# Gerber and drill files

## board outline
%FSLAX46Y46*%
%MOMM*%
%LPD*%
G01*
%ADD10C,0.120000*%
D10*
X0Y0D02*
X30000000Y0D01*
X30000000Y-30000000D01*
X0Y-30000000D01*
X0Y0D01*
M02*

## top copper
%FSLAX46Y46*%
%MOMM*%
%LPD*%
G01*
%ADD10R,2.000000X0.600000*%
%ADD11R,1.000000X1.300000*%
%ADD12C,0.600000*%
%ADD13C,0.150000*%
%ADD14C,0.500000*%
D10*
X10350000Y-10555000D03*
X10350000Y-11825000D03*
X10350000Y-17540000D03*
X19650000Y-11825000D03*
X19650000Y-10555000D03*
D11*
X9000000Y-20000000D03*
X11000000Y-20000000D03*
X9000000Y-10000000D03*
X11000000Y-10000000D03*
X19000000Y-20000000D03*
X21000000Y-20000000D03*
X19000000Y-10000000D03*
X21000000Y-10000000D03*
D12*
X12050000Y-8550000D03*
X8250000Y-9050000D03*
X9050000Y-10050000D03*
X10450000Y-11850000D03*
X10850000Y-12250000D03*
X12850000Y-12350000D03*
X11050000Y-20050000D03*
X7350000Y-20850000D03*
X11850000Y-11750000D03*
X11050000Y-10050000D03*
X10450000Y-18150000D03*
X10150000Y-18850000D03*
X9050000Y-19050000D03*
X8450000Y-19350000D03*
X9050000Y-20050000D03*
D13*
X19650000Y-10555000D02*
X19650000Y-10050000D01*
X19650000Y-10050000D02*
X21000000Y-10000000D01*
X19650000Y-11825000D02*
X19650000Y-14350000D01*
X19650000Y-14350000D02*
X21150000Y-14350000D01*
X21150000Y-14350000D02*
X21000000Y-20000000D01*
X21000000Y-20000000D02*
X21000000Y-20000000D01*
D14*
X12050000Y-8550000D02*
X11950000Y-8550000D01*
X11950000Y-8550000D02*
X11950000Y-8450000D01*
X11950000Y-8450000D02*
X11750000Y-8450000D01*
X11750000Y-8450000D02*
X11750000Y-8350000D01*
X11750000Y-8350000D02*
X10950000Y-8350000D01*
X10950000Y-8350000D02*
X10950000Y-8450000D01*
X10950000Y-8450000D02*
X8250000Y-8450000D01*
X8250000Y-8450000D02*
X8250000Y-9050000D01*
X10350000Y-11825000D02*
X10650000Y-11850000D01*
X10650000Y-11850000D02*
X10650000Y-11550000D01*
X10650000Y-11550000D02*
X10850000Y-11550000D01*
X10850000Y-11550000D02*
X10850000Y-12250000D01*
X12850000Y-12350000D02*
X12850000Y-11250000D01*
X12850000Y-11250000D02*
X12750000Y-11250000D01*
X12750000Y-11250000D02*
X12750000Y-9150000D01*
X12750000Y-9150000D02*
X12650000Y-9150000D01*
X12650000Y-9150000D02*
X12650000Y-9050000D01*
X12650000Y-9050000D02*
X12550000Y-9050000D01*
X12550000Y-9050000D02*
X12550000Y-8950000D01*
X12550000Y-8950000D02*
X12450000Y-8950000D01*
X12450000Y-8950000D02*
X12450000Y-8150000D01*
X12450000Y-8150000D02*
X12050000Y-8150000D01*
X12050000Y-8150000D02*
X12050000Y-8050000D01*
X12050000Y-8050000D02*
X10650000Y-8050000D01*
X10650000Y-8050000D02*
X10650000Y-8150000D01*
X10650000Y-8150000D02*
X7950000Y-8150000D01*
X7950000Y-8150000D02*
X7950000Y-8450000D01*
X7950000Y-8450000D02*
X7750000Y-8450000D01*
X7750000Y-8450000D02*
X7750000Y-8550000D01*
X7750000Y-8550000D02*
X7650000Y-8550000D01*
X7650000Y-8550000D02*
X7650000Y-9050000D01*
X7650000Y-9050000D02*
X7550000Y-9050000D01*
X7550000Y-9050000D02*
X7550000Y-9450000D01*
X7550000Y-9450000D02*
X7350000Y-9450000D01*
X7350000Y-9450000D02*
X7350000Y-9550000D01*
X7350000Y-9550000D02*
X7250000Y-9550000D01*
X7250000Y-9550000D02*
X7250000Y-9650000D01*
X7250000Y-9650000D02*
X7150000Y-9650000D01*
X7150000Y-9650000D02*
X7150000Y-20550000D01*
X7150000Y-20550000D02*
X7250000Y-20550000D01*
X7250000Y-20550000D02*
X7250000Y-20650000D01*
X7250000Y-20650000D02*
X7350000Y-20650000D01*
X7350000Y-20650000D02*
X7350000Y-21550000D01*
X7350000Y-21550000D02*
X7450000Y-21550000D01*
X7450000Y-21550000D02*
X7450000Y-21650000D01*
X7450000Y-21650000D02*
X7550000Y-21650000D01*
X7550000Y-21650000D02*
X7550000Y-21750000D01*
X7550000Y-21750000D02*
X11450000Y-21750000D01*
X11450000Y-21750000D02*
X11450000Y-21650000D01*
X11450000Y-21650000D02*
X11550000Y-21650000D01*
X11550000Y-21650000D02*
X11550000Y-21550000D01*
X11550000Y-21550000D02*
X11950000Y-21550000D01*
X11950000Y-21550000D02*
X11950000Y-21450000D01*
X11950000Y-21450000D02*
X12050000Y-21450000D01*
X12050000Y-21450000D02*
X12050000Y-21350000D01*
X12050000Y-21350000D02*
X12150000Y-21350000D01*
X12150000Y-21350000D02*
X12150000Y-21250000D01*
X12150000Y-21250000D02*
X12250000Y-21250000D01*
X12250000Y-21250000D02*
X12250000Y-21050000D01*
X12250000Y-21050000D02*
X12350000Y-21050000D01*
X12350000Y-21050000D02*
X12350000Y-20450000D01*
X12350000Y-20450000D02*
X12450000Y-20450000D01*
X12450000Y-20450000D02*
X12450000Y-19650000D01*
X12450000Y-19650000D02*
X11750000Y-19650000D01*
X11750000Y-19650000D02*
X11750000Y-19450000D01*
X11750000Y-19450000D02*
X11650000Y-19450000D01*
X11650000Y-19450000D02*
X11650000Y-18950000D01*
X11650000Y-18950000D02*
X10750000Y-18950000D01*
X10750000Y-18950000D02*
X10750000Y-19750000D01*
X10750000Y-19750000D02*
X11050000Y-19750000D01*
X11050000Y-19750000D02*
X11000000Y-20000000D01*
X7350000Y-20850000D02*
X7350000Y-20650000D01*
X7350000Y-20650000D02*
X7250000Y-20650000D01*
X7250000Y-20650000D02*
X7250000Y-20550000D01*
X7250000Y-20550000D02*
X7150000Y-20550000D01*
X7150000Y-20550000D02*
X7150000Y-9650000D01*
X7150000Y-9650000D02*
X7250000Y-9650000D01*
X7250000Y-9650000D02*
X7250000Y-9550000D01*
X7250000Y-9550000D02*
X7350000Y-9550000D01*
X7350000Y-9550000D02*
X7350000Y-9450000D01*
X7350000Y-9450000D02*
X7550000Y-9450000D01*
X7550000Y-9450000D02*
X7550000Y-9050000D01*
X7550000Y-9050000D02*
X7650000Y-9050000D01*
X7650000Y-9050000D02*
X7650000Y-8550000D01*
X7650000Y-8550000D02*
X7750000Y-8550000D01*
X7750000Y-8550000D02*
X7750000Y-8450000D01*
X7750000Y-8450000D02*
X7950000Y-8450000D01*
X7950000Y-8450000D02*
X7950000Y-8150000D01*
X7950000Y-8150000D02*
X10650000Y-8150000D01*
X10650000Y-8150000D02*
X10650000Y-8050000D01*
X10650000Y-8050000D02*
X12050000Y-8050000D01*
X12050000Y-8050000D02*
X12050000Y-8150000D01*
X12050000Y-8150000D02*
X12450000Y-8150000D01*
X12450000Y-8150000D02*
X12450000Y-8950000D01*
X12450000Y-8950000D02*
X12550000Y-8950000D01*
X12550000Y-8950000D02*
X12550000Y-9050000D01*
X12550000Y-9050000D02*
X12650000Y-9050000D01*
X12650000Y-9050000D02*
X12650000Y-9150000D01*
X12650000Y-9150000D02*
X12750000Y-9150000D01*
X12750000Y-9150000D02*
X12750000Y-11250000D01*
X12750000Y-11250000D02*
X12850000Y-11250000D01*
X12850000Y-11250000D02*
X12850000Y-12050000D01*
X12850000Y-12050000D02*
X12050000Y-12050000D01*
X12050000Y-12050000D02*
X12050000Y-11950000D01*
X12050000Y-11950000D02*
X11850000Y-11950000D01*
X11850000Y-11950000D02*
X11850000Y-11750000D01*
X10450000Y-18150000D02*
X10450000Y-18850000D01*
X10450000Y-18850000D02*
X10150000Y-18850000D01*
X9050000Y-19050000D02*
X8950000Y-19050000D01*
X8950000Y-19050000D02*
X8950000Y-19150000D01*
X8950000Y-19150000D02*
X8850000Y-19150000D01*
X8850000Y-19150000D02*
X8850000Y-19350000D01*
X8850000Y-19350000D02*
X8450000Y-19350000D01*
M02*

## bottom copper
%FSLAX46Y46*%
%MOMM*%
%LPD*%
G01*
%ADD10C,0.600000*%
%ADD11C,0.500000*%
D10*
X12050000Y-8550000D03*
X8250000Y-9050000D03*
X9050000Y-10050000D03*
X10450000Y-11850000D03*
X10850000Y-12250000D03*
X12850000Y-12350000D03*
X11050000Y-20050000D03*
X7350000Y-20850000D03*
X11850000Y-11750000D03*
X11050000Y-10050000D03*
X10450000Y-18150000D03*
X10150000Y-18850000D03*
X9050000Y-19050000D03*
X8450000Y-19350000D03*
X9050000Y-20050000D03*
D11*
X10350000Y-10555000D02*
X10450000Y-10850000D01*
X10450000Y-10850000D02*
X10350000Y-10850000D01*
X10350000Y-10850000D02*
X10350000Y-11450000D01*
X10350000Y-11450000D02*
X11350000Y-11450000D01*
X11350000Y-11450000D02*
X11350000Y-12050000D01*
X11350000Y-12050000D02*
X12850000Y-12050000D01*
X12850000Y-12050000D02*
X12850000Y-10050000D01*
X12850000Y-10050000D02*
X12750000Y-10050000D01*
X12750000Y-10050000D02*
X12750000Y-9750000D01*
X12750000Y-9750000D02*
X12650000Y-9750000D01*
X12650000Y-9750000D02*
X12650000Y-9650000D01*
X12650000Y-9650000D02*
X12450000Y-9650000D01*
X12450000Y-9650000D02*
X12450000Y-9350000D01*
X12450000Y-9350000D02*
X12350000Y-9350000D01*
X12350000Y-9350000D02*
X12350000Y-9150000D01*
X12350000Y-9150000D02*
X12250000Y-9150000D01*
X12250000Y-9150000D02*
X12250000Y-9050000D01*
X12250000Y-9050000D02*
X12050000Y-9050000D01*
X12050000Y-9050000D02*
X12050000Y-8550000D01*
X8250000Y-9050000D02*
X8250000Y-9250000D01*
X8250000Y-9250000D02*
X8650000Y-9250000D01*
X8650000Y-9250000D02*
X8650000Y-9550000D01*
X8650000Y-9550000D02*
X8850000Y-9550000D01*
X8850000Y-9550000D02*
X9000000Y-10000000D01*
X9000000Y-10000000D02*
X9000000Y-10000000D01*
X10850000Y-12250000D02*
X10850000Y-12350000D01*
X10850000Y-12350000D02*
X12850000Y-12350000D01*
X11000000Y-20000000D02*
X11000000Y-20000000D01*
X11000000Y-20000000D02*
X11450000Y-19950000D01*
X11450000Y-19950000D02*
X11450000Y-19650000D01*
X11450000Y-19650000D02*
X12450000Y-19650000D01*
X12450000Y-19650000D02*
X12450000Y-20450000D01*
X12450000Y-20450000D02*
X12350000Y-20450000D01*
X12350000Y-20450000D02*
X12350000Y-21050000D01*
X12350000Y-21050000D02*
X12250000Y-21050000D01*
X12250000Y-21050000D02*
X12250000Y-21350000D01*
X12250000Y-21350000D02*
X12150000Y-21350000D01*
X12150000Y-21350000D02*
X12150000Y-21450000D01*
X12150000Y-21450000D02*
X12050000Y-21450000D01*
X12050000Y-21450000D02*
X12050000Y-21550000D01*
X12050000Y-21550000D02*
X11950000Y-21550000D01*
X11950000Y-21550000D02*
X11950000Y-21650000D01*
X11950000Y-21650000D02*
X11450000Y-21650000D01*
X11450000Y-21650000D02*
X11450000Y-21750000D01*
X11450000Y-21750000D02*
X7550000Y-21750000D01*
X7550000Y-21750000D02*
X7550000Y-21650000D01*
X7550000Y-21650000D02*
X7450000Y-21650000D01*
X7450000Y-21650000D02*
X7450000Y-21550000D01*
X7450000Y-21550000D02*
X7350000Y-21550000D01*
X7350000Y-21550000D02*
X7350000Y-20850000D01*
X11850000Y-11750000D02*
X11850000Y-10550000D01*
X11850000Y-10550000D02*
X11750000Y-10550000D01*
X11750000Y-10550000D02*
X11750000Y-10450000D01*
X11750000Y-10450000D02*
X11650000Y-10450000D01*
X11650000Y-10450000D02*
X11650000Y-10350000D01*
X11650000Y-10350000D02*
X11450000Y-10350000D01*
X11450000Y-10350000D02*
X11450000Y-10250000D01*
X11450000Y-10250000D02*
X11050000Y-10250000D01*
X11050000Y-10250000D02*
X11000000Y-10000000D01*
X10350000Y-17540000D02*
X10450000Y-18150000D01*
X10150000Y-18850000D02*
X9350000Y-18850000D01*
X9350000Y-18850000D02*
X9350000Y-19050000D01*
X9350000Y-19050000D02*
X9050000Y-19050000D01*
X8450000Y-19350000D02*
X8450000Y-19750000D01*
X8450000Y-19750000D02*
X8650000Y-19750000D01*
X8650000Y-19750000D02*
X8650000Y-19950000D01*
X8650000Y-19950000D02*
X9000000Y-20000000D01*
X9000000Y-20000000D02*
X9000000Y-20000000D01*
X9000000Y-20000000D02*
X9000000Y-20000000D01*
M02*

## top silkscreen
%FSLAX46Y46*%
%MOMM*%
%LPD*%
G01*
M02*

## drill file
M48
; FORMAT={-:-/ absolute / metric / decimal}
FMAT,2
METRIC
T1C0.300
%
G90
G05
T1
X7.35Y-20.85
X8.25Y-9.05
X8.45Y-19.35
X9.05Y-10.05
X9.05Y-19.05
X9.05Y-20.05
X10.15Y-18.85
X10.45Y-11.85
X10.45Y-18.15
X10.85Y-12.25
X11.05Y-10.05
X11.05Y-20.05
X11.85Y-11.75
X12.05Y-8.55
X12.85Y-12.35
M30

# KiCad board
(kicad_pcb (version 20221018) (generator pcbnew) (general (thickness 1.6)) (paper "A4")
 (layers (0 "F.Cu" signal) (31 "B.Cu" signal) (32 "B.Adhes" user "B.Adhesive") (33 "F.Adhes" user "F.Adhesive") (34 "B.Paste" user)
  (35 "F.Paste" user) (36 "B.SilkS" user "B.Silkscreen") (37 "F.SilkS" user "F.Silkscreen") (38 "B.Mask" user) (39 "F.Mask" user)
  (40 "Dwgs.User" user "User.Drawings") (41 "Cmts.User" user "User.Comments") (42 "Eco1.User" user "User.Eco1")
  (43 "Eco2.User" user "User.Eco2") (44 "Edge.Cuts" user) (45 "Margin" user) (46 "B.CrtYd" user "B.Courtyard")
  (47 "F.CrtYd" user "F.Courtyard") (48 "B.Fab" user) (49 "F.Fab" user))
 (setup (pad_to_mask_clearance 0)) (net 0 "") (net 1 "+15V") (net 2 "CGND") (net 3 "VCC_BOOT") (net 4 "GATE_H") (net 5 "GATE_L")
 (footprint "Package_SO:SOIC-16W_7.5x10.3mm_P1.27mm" (layer "F.Cu") (at 15 14.999999656677247 0) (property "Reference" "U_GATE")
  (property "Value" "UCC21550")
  (pad "1" smd rect (at -4.65 -4.445) (size 2 0.6) (layers "F.Cu" "F.Paste" "F.Mask") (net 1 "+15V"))
  (pad "2" smd rect (at -4.65 -3.175) (size 2 0.6) (layers "F.Cu" "F.Paste" "F.Mask") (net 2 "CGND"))
  (pad "7" smd rect (at -4.65 2.54) (size 2 0.6) (layers "F.Cu" "F.Paste" "F.Mask") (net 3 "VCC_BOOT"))
  (pad "14" smd rect (at 4.65 -3.175) (size 2 0.6) (layers "F.Cu" "F.Paste" "F.Mask") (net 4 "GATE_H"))
  (pad "16" smd rect (at 4.65 -4.445) (size 2 0.6) (layers "F.Cu" "F.Paste" "F.Mask") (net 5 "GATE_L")))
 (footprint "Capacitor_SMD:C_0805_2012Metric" (layer "F.Cu") (at 10 20 0) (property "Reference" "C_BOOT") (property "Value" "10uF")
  (pad "1" smd rect (at -1 0) (size 1 1.3) (layers "F.Cu" "F.Paste" "F.Mask") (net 3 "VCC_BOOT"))
  (pad "2" smd rect (at 1 0) (size 1 1.3) (layers "F.Cu" "F.Paste" "F.Mask") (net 2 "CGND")))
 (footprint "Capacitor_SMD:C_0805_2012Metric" (layer "F.Cu") (at 10 10 0) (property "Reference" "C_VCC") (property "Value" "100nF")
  (pad "1" smd rect (at -1 0) (size 1 1.3) (layers "F.Cu" "F.Paste" "F.Mask") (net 1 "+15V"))
  (pad "2" smd rect (at 1 0) (size 1 1.3) (layers "F.Cu" "F.Paste" "F.Mask") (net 2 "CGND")))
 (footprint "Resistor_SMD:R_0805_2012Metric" (layer "F.Cu") (at 20 20 0) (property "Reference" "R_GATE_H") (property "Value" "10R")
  (pad "1" smd rect (at -1 0) (size 1 1.3) (layers "F.Cu" "F.Paste" "F.Mask") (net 4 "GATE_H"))
  (pad "2" smd rect (at 1 0) (size 1 1.3) (layers "F.Cu" "F.Paste" "F.Mask") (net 4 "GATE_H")))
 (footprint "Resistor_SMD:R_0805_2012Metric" (layer "F.Cu") (at 20 10 0) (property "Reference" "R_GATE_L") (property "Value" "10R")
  (pad "1" smd rect (at -1 0) (size 1 1.3) (layers "F.Cu" "F.Paste" "F.Mask") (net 5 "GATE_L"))
  (pad "2" smd rect (at 1 0) (size 1 1.3) (layers "F.Cu" "F.Paste" "F.Mask") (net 5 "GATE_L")))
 (gr_rect (start 0 0) (end 30 30) (layer "Edge.Cuts") (width 0.12))
 (segment (start 19.65 10.554999656677246) (end 19.650000000000002 10.05) (width 0.15) (layer "F.Cu") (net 5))
 (segment (start 19.650000000000002 10.05) (end 21.0 10.0) (width 0.15) (layer "F.Cu") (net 5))
 (segment (start 19.65 11.824999656677246) (end 19.650000000000002 14.350000000000001) (width 0.15) (layer "F.Cu") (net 4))
 (segment (start 19.650000000000002 14.350000000000001) (end 21.150000000000002 14.350000000000001) (width 0.15) (layer "F.Cu") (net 4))
 (segment (start 21.150000000000002 14.350000000000001) (end 21.0 20.0) (width 0.15) (layer "F.Cu") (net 4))
 (segment (start 21.0 20.0) (end 21.0 20.0) (width 0.15) (layer "F.Cu") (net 4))
 (segment (start 10.35 10.554999656677246) (end 10.450000000000001 10.850000000000001) (width 0.5) (layer "B.Cu") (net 1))
 (segment (start 10.450000000000001 10.850000000000001) (end 10.350000000000001 10.850000000000001) (width 0.5) (layer "B.Cu") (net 1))
 (segment (start 10.350000000000001 10.850000000000001) (end 10.350000000000001 11.450000000000001) (width 0.5) (layer "B.Cu") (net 1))
 (segment (start 10.350000000000001 11.450000000000001) (end 11.350000000000001 11.450000000000001) (width 0.5) (layer "B.Cu") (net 1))
 (segment (start 11.350000000000001 11.450000000000001) (end 11.350000000000001 12.05) (width 0.5) (layer "B.Cu") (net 1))
 (segment (start 11.350000000000001 12.05) (end 12.850000000000001 12.05) (width 0.5) (layer "B.Cu") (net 1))
 (segment (start 12.850000000000001 12.05) (end 12.850000000000001 10.05) (width 0.5) (layer "B.Cu") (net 1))
 (segment (start 12.850000000000001 10.05) (end 12.750000000000002 10.05) (width 0.5) (layer "B.Cu") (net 1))
 (segment (start 12.750000000000002 10.05) (end 12.750000000000002 9.750000000000002) (width 0.5) (layer "B.Cu") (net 1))
 (segment (start 12.750000000000002 9.750000000000002) (end 12.650000000000002 9.750000000000002) (width 0.5) (layer "B.Cu") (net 1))
 (segment (start 12.650000000000002 9.750000000000002) (end 12.650000000000002 9.650000000000002) (width 0.5) (layer "B.Cu") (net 1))
 (segment (start 12.650000000000002 9.650000000000002) (end 12.450000000000001 9.650000000000002) (width 0.5) (layer "B.Cu") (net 1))
 (segment (start 12.450000000000001 9.650000000000002) (end 12.450000000000001 9.350000000000001) (width 0.5) (layer "B.Cu") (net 1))
 (segment (start 12.450000000000001 9.350000000000001) (end 12.350000000000001 9.350000000000001) (width 0.5) (layer "B.Cu") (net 1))
 (segment (start 12.350000000000001 9.350000000000001) (end 12.350000000000001 9.15) (width 0.5) (layer "B.Cu") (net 1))
 (segment (start 12.350000000000001 9.15) (end 12.250000000000002 9.15) (width 0.5) (layer "B.Cu") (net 1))
 (segment (start 12.250000000000002 9.15) (end 12.250000000000002 9.05) (width 0.5) (layer "B.Cu") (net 1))
 (segment (start 12.250000000000002 9.05) (end 12.05 9.05) (width 0.5) (layer "B.Cu") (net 1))
 (segment (start 12.05 9.05) (end 12.05 8.55) (width 0.5) (layer "B.Cu") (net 1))
 (segment (start 12.05 8.55) (end 11.950000000000001 8.55) (width 0.5) (layer "F.Cu") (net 1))
 (segment (start 11.950000000000001 8.55) (end 11.950000000000001 8.450000000000001) (width 0.5) (layer "F.Cu") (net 1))
 (segment (start 11.950000000000001 8.450000000000001) (end 11.750000000000002 8.450000000000001) (width 0.5) (layer "F.Cu") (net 1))
 (segment (start 11.750000000000002 8.450000000000001) (end 11.750000000000002 8.350000000000001) (width 0.5) (layer "F.Cu") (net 1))
 (segment (start 11.750000000000002 8.350000000000001) (end 10.950000000000001 8.350000000000001) (width 0.5) (layer "F.Cu") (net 1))
 (segment (start 10.950000000000001 8.350000000000001) (end 10.950000000000001 8.450000000000001) (width 0.5) (layer "F.Cu") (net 1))
 (segment (start 10.950000000000001 8.450000000000001) (end 8.250000000000002 8.450000000000001) (width 0.5) (layer "F.Cu") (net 1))
 (segment (start 8.250000000000002 8.450000000000001) (end 8.250000000000002 9.05) (width 0.5) (layer "F.Cu") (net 1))
 (segment (start 8.250000000000002 9.05) (end 8.250000000000002 9.250000000000002) (width 0.5) (layer "B.Cu") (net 1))
 (segment (start 8.250000000000002 9.250000000000002) (end 8.65 9.250000000000002) (width 0.5) (layer "B.Cu") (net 1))
 (segment (start 8.65 9.250000000000002) (end 8.65 9.55) (width 0.5) (layer "B.Cu") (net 1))
 (segment (start 8.65 9.55) (end 8.850000000000001 9.55) (width 0.5) (layer "B.Cu") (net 1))
 (segment (start 8.850000000000001 9.55) (end 9.0 10.0) (width 0.5) (layer "B.Cu") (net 1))
 (segment (start 9.0 10.0) (end 9.0 10.0) (width 0.5) (layer "B.Cu") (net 1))
 (segment (start 10.35 11.824999656677246) (end 10.650000000000002 11.850000000000001) (width 0.5) (layer "F.Cu") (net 2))
 (segment (start 10.650000000000002 11.850000000000001) (end 10.650000000000002 11.55) (width 0.5) (layer "F.Cu") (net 2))
 (segment (start 10.650000000000002 11.55) (end 10.850000000000001 11.55) (width 0.5) (layer "F.Cu") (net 2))
 (segment (start 10.850000000000001 11.55) (end 10.850000000000001 12.250000000000002) (width 0.5) (layer "F.Cu") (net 2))
 (segment (start 10.850000000000001 12.250000000000002) (end 10.850000000000001 12.350000000000001) (width 0.5) (layer "B.Cu") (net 2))
 (segment (start 10.850000000000001 12.350000000000001) (end 12.850000000000001 12.350000000000001) (width 0.5) (layer "B.Cu") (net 2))
 (segment (start 12.850000000000001 12.350000000000001) (end 12.850000000000001 11.250000000000002) (width 0.5) (layer "F.Cu") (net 2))
 (segment (start 12.850000000000001 11.250000000000002) (end 12.750000000000002 11.250000000000002) (width 0.5) (layer "F.Cu") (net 2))
 (segment (start 12.750000000000002 11.250000000000002) (end 12.750000000000002 9.15) (width 0.5) (layer "F.Cu") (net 2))
 (segment (start 12.750000000000002 9.15) (end 12.650000000000002 9.15) (width 0.5) (layer "F.Cu") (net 2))
 (segment (start 12.650000000000002 9.15) (end 12.650000000000002 9.05) (width 0.5) (layer "F.Cu") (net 2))
 (segment (start 12.650000000000002 9.05) (end 12.55 9.05) (width 0.5) (layer "F.Cu") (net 2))
 (segment (start 12.55 9.05) (end 12.55 8.950000000000001) (width 0.5) (layer "F.Cu") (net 2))
 (segment (start 12.55 8.950000000000001) (end 12.450000000000001 8.950000000000001) (width 0.5) (layer "F.Cu") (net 2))
 (segment (start 12.450000000000001 8.950000000000001) (end 12.450000000000001 8.15) (width 0.5) (layer "F.Cu") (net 2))
 (segment (start 12.450000000000001 8.15) (end 12.05 8.15) (width 0.5) (layer "F.Cu") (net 2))
 (segment (start 12.05 8.15) (end 12.05 8.05) (width 0.5) (layer "F.Cu") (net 2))
 (segment (start 12.05 8.05) (end 10.650000000000002 8.05) (width 0.5) (layer "F.Cu") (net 2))
 (segment (start 10.650000000000002 8.05) (end 10.650000000000002 8.15) (width 0.5) (layer "F.Cu") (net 2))
 (segment (start 10.650000000000002 8.15) (end 7.95 8.15) (width 0.5) (layer "F.Cu") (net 2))
 (segment (start 7.95 8.15) (end 7.95 8.450000000000001) (width 0.5) (layer "F.Cu") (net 2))
 (segment (start 7.95 8.450000000000001) (end 7.75 8.450000000000001) (width 0.5) (layer "F.Cu") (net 2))
 (segment (start 7.75 8.450000000000001) (end 7.75 8.55) (width 0.5) (layer "F.Cu") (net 2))
 (segment (start 7.75 8.55) (end 7.65 8.55) (width 0.5) (layer "F.Cu") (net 2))
 (segment (start 7.65 8.55) (end 7.65 9.05) (width 0.5) (layer "F.Cu") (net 2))
 (segment (start 7.65 9.05) (end 7.55 9.05) (width 0.5) (layer "F.Cu") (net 2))
 (segment (start 7.55 9.05) (end 7.55 9.450000000000001) (width 0.5) (layer "F.Cu") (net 2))
 (segment (start 7.55 9.450000000000001) (end 7.3500000000000005 9.450000000000001) (width 0.5) (layer "F.Cu") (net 2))
 (segment (start 7.3500000000000005 9.450000000000001) (end 7.3500000000000005 9.55) (width 0.5) (layer "F.Cu") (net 2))
 (segment (start 7.3500000000000005 9.55) (end 7.25 9.55) (width 0.5) (layer "F.Cu") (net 2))
 (segment (start 7.25 9.55) (end 7.25 9.650000000000002) (width 0.5) (layer "F.Cu") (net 2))
 (segment (start 7.25 9.650000000000002) (end 7.15 9.650000000000002) (width 0.5) (layer "F.Cu") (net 2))
 (segment (start 7.15 9.650000000000002) (end 7.15 20.55) (width 0.5) (layer "F.Cu") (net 2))
 (segment (start 7.15 20.55) (end 7.25 20.55) (width 0.5) (layer "F.Cu") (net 2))
 (segment (start 7.25 20.55) (end 7.25 20.650000000000002) (width 0.5) (layer "F.Cu") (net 2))
 (segment (start 7.25 20.650000000000002) (end 7.3500000000000005 20.650000000000002) (width 0.5) (layer "F.Cu") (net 2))
 (segment (start 7.3500000000000005 20.650000000000002) (end 7.3500000000000005 21.55) (width 0.5) (layer "F.Cu") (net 2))
 (segment (start 7.3500000000000005 21.55) (end 7.45 21.55) (width 0.5) (layer "F.Cu") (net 2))
 (segment (start 7.45 21.55) (end 7.45 21.650000000000002) (width 0.5) (layer "F.Cu") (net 2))
 (segment (start 7.45 21.650000000000002) (end 7.55 21.650000000000002) (width 0.5) (layer "F.Cu") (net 2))
 (segment (start 7.55 21.650000000000002) (end 7.55 21.750000000000004) (width 0.5) (layer "F.Cu") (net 2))
 (segment (start 7.55 21.750000000000004) (end 11.450000000000001 21.750000000000004) (width 0.5) (layer "F.Cu") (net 2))
 (segment (start 11.450000000000001 21.750000000000004) (end 11.450000000000001 21.650000000000002) (width 0.5) (layer "F.Cu") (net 2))
 (segment (start 11.450000000000001 21.650000000000002) (end 11.55 21.650000000000002) (width 0.5) (layer "F.Cu") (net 2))
 (segment (start 11.55 21.650000000000002) (end 11.55 21.55) (width 0.5) (layer "F.Cu") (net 2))
 (segment (start 11.55 21.55) (end 11.950000000000001 21.55) (width 0.5) (layer "F.Cu") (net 2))
 (segment (start 11.950000000000001 21.55) (end 11.950000000000001 21.450000000000003) (width 0.5) (layer "F.Cu") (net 2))
 (segment (start 11.950000000000001 21.450000000000003) (end 12.05 21.450000000000003) (width 0.5) (layer "F.Cu") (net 2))
 (segment (start 12.05 21.450000000000003) (end 12.05 21.35) (width 0.5) (layer "F.Cu") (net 2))
 (segment (start 12.05 21.35) (end 12.150000000000002 21.35) (width 0.5) (layer "F.Cu") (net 2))
 (segment (start 12.150000000000002 21.35) (end 12.150000000000002 21.250000000000004) (width 0.5) (layer "F.Cu") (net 2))
 (segment (start 12.150000000000002 21.250000000000004) (end 12.250000000000002 21.250000000000004) (width 0.5) (layer "F.Cu") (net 2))
 (segment (start 12.250000000000002 21.250000000000004) (end 12.250000000000002 21.05) (width 0.5) (layer "F.Cu") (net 2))
 (segment (start 12.250000000000002 21.05) (end 12.350000000000001 21.05) (width 0.5) (layer "F.Cu") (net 2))
 (segment (start 12.350000000000001 21.05) (end 12.350000000000001 20.450000000000003) (width 0.5) (layer "F.Cu") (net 2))
 (segment (start 12.350000000000001 20.450000000000003) (end 12.450000000000001 20.450000000000003) (width 0.5) (layer "F.Cu") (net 2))
 (segment (start 12.450000000000001 20.450000000000003) (end 12.450000000000001 19.650000000000002) (width 0.5) (layer "F.Cu") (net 2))
 (segment (start 12.450000000000001 19.650000000000002) (end 11.750000000000002 19.650000000000002) (width 0.5) (layer "F.Cu") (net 2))
 (segment (start 11.750000000000002 19.650000000000002) (end 11.750000000000002 19.450000000000003) (width 0.5) (layer "F.Cu") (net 2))
 (segment (start 11.750000000000002 19.450000000000003) (end 11.650000000000002 19.450000000000003) (width 0.5) (layer "F.Cu") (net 2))
 (segment (start 11.650000000000002 19.450000000000003) (end 11.650000000000002 18.950000000000003) (width 0.5) (layer "F.Cu") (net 2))
 (segment (start 11.650000000000002 18.950000000000003) (end 10.750000000000002 18.950000000000003) (width 0.5) (layer "F.Cu") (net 2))
 (segment (start 10.750000000000002 18.950000000000003) (end 10.750000000000002 19.750000000000004) (width 0.5) (layer "F.Cu") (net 2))
 (segment (start 10.750000000000002 19.750000000000004) (end 11.05 19.750000000000004) (width 0.5) (layer "F.Cu") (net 2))
 (segment (start 11.05 19.750000000000004) (end 11.0 20.0) (width 0.5) (layer "F.Cu") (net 2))
 (segment (start 11.0 20.0) (end 11.0 20.0) (width 0.5) (layer "B.Cu") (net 2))
 (segment (start 11.0 20.0) (end 11.450000000000001 19.950000000000003) (width 0.5) (layer "B.Cu") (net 2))
 (segment (start 11.450000000000001 19.950000000000003) (end 11.450000000000001 19.650000000000002) (width 0.5) (layer "B.Cu") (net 2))
 (segment (start 11.450000000000001 19.650000000000002) (end 12.450000000000001 19.650000000000002) (width 0.5) (layer "B.Cu") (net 2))
 (segment (start 12.450000000000001 19.650000000000002) (end 12.450000000000001 20.450000000000003) (width 0.5) (layer "B.Cu") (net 2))
 (segment (start 12.450000000000001 20.450000000000003) (end 12.350000000000001 20.450000000000003) (width 0.5) (layer "B.Cu") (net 2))
 (segment (start 12.350000000000001 20.450000000000003) (end 12.350000000000001 21.05) (width 0.5) (layer "B.Cu") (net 2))
 (segment (start 12.350000000000001 21.05) (end 12.250000000000002 21.05) (width 0.5) (layer "B.Cu") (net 2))
 (segment (start 12.250000000000002 21.05) (end 12.250000000000002 21.35) (width 0.5) (layer "B.Cu") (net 2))
 (segment (start 12.250000000000002 21.35) (end 12.150000000000002 21.35) (width 0.5) (layer "B.Cu") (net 2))
 (segment (start 12.150000000000002 21.35) (end 12.150000000000002 21.450000000000003) (width 0.5) (layer "B.Cu") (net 2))
 (segment (start 12.150000000000002 21.450000000000003) (end 12.05 21.450000000000003) (width 0.5) (layer "B.Cu") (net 2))
 (segment (start 12.05 21.450000000000003) (end 12.05 21.55) (width 0.5) (layer "B.Cu") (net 2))
 (segment (start 12.05 21.55) (end 11.950000000000001 21.55) (width 0.5) (layer "B.Cu") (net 2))
 (segment (start 11.950000000000001 21.55) (end 11.950000000000001 21.650000000000002) (width 0.5) (layer "B.Cu") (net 2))
 (segment (start 11.950000000000001 21.650000000000002) (end 11.450000000000001 21.650000000000002) (width 0.5) (layer "B.Cu") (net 2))
 (segment (start 11.450000000000001 21.650000000000002) (end 11.450000000000001 21.750000000000004) (width 0.5) (layer "B.Cu") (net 2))
 (segment (start 11.450000000000001 21.750000000000004) (end 7.55 21.750000000000004) (width 0.5) (layer "B.Cu") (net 2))
 (segment (start 7.55 21.750000000000004) (end 7.55 21.650000000000002) (width 0.5) (layer "B.Cu") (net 2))
 (segment (start 7.55 21.650000000000002) (end 7.45 21.650000000000002) (width 0.5) (layer "B.Cu") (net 2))
 (segment (start 7.45 21.650000000000002) (end 7.45 21.55) (width 0.5) (layer "B.Cu") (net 2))
 (segment (start 7.45 21.55) (end 7.3500000000000005 21.55) (width 0.5) (layer "B.Cu") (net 2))
 (segment (start 7.3500000000000005 21.55) (end 7.3500000000000005 20.85) (width 0.5) (layer "B.Cu") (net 2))
 (segment (start 7.3500000000000005 20.85) (end 7.3500000000000005 20.650000000000002) (width 0.5) (layer "F.Cu") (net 2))
 (segment (start 7.3500000000000005 20.650000000000002) (end 7.25 20.650000000000002) (width 0.5) (layer "F.Cu") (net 2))
 (segment (start 7.25 20.650000000000002) (end 7.25 20.55) (width 0.5) (layer "F.Cu") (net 2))
 (segment (start 7.25 20.55) (end 7.15 20.55) (width 0.5) (layer "F.Cu") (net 2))
 (segment (start 7.15 20.55) (end 7.15 9.650000000000002) (width 0.5) (layer "F.Cu") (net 2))
 (segment (start 7.15 9.650000000000002) (end 7.25 9.650000000000002) (width 0.5) (layer "F.Cu") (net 2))
 (segment (start 7.25 9.650000000000002) (end 7.25 9.55) (width 0.5) (layer "F.Cu") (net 2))
 (segment (start 7.25 9.55) (end 7.3500000000000005 9.55) (width 0.5) (layer "F.Cu") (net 2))
 (segment (start 7.3500000000000005 9.55) (end 7.3500000000000005 9.450000000000001) (width 0.5) (layer "F.Cu") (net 2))
 (segment (start 7.3500000000000005 9.450000000000001) (end 7.55 9.450000000000001) (width 0.5) (layer "F.Cu") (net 2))
 (segment (start 7.55 9.450000000000001) (end 7.55 9.05) (width 0.5) (layer "F.Cu") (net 2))
 (segment (start 7.55 9.05) (end 7.65 9.05) (width 0.5) (layer "F.Cu") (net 2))
 (segment (start 7.65 9.05) (end 7.65 8.55) (width 0.5) (layer "F.Cu") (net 2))
 (segment (start 7.65 8.55) (end 7.75 8.55) (width 0.5) (layer "F.Cu") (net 2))
 (segment (start 7.75 8.55) (end 7.75 8.450000000000001) (width 0.5) (layer "F.Cu") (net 2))
 (segment (start 7.75 8.450000000000001) (end 7.95 8.450000000000001) (width 0.5) (layer "F.Cu") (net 2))
 (segment (start 7.95 8.450000000000001) (end 7.95 8.15) (width 0.5) (layer "F.Cu") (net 2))
 (segment (start 7.95 8.15) (end 10.650000000000002 8.15) (width 0.5) (layer "F.Cu") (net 2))
 (segment (start 10.650000000000002 8.15) (end 10.650000000000002 8.05) (width 0.5) (layer "F.Cu") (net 2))
 (segment (start 10.650000000000002 8.05) (end 12.05 8.05) (width 0.5) (layer "F.Cu") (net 2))
 (segment (start 12.05 8.05) (end 12.05 8.15) (width 0.5) (layer "F.Cu") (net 2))
 (segment (start 12.05 8.15) (end 12.450000000000001 8.15) (width 0.5) (layer "F.Cu") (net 2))
 (segment (start 12.450000000000001 8.15) (end 12.450000000000001 8.950000000000001) (width 0.5) (layer "F.Cu") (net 2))
 (segment (start 12.450000000000001 8.950000000000001) (end 12.55 8.950000000000001) (width 0.5) (layer "F.Cu") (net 2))
 (segment (start 12.55 8.950000000000001) (end 12.55 9.05) (width 0.5) (layer "F.Cu") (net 2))
 (segment (start 12.55 9.05) (end 12.650000000000002 9.05) (width 0.5) (layer "F.Cu") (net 2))
 (segment (start 12.650000000000002 9.05) (end 12.650000000000002 9.15) (width 0.5) (layer "F.Cu") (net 2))
 (segment (start 12.650000000000002 9.15) (end 12.750000000000002 9.15) (width 0.5) (layer "F.Cu") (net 2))
 (segment (start 12.750000000000002 9.15) (end 12.750000000000002 11.250000000000002) (width 0.5) (layer "F.Cu") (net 2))
 (segment (start 12.750000000000002 11.250000000000002) (end 12.850000000000001 11.250000000000002) (width 0.5) (layer "F.Cu") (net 2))
 (segment (start 12.850000000000001 11.250000000000002) (end 12.850000000000001 12.05) (width 0.5) (layer "F.Cu") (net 2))
 (segment (start 12.850000000000001 12.05) (end 12.05 12.05) (width 0.5) (layer "F.Cu") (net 2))
 (segment (start 12.05 12.05) (end 12.05 11.950000000000001) (width 0.5) (layer "F.Cu") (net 2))
 (segment (start 12.05 11.950000000000001) (end 11.850000000000001 11.950000000000001) (width 0.5) (layer "F.Cu") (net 2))
 (segment (start 11.850000000000001 11.950000000000001) (end 11.850000000000001 11.750000000000002) (width 0.5) (layer "F.Cu") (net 2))
 (segment (start 11.850000000000001 11.750000000000002) (end 11.850000000000001 10.55) (width 0.5) (layer "B.Cu") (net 2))
 (segment (start 11.850000000000001 10.55) (end 11.750000000000002 10.55) (width 0.5) (layer "B.Cu") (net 2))
 (segment (start 11.750000000000002 10.55) (end 11.750000000000002 10.450000000000001) (width 0.5) (layer "B.Cu") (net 2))
 (segment (start 11.750000000000002 10.450000000000001) (end 11.650000000000002 10.450000000000001) (width 0.5) (layer "B.Cu") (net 2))
 (segment (start 11.650000000000002 10.450000000000001) (end 11.650000000000002 10.350000000000001) (width 0.5) (layer "B.Cu") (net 2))
 (segment (start 11.650000000000002 10.350000000000001) (end 11.450000000000001 10.350000000000001) (width 0.5) (layer "B.Cu") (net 2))
 (segment (start 11.450000000000001 10.350000000000001) (end 11.450000000000001 10.250000000000002) (width 0.5) (layer "B.Cu") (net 2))
 (segment (start 11.450000000000001 10.250000000000002) (end 11.05 10.250000000000002) (width 0.5) (layer "B.Cu") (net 2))
 (segment (start 11.05 10.250000000000002) (end 11.0 10.0) (width 0.5) (layer "B.Cu") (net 2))
 (segment (start 10.35 17.539999656677246) (end 10.450000000000001 18.150000000000002) (width 0.5) (layer "B.Cu") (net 3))
 (segment (start 10.450000000000001 18.150000000000002) (end 10.450000000000001 18.85) (width 0.5) (layer "F.Cu") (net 3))
 (segment (start 10.450000000000001 18.85) (end 10.150000000000002 18.85) (width 0.5) (layer "F.Cu") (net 3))
 (segment (start 10.150000000000002 18.85) (end 9.350000000000001 18.85) (width 0.5) (layer "B.Cu") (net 3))
 (segment (start 9.350000000000001 18.85) (end 9.350000000000001 19.05) (width 0.5) (layer "B.Cu") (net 3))
 (segment (start 9.350000000000001 19.05) (end 9.05 19.05) (width 0.5) (layer "B.Cu") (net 3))
 (segment (start 9.05 19.05) (end 8.950000000000001 19.05) (width 0.5) (layer "F.Cu") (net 3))
 (segment (start 8.950000000000001 19.05) (end 8.950000000000001 19.150000000000002) (width 0.5) (layer "F.Cu") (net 3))
 (segment (start 8.950000000000001 19.150000000000002) (end 8.850000000000001 19.150000000000002) (width 0.5) (layer "F.Cu") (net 3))
 (segment (start 8.850000000000001 19.150000000000002) (end 8.850000000000001 19.35) (width 0.5) (layer "F.Cu") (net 3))
 (segment (start 8.850000000000001 19.35) (end 8.450000000000001 19.35) (width 0.5) (layer "F.Cu") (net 3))
 (segment (start 8.450000000000001 19.35) (end 8.450000000000001 19.750000000000004) (width 0.5) (layer "B.Cu") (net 3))
 (segment (start 8.450000000000001 19.750000000000004) (end 8.65 19.750000000000004) (width 0.5) (layer "B.Cu") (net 3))
 (segment (start 8.65 19.750000000000004) (end 8.65 19.950000000000003) (width 0.5) (layer "B.Cu") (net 3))
 (segment (start 8.65 19.950000000000003) (end 9.0 20.0) (width 0.5) (layer "B.Cu") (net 3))
 (segment (start 9.0 20.0) (end 9.0 20.0) (width 0.5) (layer "B.Cu") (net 3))
 (segment (start 9.0 20.0) (end 9.0 20.0) (width 0.5) (layer "B.Cu") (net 3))
 (via (at 12.05 8.55) (size 0.6) (drill 0.3) (layers "B.Cu" "F.Cu") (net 1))
 (via (at 8.250000000000002 9.05) (size 0.6) (drill 0.3) (layers "B.Cu" "F.Cu") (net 1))
 (via (at 9.05 10.05) (size 0.6) (drill 0.3) (layers "B.Cu" "F.Cu") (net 1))
 (via (at 10.450000000000001 11.850000000000001) (size 0.6) (drill 0.3) (layers "B.Cu" "F.Cu") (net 2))
 (via (at 10.850000000000001 12.250000000000002) (size 0.6) (drill 0.3) (layers "B.Cu" "F.Cu") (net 2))
 (via (at 12.850000000000001 12.350000000000001) (size 0.6) (drill 0.3) (layers "B.Cu" "F.Cu") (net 2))
 (via (at 11.05 20.05) (size 0.6) (drill 0.3) (layers "B.Cu" "F.Cu") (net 2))
 (via (at 7.3500000000000005 20.85) (size 0.6) (drill 0.3) (layers "B.Cu" "F.Cu") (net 2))
 (via (at 11.850000000000001 11.750000000000002) (size 0.6) (drill 0.3) (layers "B.Cu" "F.Cu") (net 2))
 (via (at 11.05 10.05) (size 0.6) (drill 0.3) (layers "B.Cu" "F.Cu") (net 2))
 (via (at 10.450000000000001 18.150000000000002) (size 0.6) (drill 0.3) (layers "B.Cu" "F.Cu") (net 3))
 (via (at 10.150000000000002 18.85) (size 0.6) (drill 0.3) (layers "B.Cu" "F.Cu") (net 3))
 (via (at 9.05 19.05) (size 0.6) (drill 0.3) (layers "B.Cu" "F.Cu") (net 3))
 (via (at 8.450000000000001 19.35) (size 0.6) (drill 0.3) (layers "B.Cu" "F.Cu") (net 3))
 (via (at 9.05 20.05) (size 0.6) (drill 0.3) (layers "B.Cu" "F.Cu") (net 3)))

